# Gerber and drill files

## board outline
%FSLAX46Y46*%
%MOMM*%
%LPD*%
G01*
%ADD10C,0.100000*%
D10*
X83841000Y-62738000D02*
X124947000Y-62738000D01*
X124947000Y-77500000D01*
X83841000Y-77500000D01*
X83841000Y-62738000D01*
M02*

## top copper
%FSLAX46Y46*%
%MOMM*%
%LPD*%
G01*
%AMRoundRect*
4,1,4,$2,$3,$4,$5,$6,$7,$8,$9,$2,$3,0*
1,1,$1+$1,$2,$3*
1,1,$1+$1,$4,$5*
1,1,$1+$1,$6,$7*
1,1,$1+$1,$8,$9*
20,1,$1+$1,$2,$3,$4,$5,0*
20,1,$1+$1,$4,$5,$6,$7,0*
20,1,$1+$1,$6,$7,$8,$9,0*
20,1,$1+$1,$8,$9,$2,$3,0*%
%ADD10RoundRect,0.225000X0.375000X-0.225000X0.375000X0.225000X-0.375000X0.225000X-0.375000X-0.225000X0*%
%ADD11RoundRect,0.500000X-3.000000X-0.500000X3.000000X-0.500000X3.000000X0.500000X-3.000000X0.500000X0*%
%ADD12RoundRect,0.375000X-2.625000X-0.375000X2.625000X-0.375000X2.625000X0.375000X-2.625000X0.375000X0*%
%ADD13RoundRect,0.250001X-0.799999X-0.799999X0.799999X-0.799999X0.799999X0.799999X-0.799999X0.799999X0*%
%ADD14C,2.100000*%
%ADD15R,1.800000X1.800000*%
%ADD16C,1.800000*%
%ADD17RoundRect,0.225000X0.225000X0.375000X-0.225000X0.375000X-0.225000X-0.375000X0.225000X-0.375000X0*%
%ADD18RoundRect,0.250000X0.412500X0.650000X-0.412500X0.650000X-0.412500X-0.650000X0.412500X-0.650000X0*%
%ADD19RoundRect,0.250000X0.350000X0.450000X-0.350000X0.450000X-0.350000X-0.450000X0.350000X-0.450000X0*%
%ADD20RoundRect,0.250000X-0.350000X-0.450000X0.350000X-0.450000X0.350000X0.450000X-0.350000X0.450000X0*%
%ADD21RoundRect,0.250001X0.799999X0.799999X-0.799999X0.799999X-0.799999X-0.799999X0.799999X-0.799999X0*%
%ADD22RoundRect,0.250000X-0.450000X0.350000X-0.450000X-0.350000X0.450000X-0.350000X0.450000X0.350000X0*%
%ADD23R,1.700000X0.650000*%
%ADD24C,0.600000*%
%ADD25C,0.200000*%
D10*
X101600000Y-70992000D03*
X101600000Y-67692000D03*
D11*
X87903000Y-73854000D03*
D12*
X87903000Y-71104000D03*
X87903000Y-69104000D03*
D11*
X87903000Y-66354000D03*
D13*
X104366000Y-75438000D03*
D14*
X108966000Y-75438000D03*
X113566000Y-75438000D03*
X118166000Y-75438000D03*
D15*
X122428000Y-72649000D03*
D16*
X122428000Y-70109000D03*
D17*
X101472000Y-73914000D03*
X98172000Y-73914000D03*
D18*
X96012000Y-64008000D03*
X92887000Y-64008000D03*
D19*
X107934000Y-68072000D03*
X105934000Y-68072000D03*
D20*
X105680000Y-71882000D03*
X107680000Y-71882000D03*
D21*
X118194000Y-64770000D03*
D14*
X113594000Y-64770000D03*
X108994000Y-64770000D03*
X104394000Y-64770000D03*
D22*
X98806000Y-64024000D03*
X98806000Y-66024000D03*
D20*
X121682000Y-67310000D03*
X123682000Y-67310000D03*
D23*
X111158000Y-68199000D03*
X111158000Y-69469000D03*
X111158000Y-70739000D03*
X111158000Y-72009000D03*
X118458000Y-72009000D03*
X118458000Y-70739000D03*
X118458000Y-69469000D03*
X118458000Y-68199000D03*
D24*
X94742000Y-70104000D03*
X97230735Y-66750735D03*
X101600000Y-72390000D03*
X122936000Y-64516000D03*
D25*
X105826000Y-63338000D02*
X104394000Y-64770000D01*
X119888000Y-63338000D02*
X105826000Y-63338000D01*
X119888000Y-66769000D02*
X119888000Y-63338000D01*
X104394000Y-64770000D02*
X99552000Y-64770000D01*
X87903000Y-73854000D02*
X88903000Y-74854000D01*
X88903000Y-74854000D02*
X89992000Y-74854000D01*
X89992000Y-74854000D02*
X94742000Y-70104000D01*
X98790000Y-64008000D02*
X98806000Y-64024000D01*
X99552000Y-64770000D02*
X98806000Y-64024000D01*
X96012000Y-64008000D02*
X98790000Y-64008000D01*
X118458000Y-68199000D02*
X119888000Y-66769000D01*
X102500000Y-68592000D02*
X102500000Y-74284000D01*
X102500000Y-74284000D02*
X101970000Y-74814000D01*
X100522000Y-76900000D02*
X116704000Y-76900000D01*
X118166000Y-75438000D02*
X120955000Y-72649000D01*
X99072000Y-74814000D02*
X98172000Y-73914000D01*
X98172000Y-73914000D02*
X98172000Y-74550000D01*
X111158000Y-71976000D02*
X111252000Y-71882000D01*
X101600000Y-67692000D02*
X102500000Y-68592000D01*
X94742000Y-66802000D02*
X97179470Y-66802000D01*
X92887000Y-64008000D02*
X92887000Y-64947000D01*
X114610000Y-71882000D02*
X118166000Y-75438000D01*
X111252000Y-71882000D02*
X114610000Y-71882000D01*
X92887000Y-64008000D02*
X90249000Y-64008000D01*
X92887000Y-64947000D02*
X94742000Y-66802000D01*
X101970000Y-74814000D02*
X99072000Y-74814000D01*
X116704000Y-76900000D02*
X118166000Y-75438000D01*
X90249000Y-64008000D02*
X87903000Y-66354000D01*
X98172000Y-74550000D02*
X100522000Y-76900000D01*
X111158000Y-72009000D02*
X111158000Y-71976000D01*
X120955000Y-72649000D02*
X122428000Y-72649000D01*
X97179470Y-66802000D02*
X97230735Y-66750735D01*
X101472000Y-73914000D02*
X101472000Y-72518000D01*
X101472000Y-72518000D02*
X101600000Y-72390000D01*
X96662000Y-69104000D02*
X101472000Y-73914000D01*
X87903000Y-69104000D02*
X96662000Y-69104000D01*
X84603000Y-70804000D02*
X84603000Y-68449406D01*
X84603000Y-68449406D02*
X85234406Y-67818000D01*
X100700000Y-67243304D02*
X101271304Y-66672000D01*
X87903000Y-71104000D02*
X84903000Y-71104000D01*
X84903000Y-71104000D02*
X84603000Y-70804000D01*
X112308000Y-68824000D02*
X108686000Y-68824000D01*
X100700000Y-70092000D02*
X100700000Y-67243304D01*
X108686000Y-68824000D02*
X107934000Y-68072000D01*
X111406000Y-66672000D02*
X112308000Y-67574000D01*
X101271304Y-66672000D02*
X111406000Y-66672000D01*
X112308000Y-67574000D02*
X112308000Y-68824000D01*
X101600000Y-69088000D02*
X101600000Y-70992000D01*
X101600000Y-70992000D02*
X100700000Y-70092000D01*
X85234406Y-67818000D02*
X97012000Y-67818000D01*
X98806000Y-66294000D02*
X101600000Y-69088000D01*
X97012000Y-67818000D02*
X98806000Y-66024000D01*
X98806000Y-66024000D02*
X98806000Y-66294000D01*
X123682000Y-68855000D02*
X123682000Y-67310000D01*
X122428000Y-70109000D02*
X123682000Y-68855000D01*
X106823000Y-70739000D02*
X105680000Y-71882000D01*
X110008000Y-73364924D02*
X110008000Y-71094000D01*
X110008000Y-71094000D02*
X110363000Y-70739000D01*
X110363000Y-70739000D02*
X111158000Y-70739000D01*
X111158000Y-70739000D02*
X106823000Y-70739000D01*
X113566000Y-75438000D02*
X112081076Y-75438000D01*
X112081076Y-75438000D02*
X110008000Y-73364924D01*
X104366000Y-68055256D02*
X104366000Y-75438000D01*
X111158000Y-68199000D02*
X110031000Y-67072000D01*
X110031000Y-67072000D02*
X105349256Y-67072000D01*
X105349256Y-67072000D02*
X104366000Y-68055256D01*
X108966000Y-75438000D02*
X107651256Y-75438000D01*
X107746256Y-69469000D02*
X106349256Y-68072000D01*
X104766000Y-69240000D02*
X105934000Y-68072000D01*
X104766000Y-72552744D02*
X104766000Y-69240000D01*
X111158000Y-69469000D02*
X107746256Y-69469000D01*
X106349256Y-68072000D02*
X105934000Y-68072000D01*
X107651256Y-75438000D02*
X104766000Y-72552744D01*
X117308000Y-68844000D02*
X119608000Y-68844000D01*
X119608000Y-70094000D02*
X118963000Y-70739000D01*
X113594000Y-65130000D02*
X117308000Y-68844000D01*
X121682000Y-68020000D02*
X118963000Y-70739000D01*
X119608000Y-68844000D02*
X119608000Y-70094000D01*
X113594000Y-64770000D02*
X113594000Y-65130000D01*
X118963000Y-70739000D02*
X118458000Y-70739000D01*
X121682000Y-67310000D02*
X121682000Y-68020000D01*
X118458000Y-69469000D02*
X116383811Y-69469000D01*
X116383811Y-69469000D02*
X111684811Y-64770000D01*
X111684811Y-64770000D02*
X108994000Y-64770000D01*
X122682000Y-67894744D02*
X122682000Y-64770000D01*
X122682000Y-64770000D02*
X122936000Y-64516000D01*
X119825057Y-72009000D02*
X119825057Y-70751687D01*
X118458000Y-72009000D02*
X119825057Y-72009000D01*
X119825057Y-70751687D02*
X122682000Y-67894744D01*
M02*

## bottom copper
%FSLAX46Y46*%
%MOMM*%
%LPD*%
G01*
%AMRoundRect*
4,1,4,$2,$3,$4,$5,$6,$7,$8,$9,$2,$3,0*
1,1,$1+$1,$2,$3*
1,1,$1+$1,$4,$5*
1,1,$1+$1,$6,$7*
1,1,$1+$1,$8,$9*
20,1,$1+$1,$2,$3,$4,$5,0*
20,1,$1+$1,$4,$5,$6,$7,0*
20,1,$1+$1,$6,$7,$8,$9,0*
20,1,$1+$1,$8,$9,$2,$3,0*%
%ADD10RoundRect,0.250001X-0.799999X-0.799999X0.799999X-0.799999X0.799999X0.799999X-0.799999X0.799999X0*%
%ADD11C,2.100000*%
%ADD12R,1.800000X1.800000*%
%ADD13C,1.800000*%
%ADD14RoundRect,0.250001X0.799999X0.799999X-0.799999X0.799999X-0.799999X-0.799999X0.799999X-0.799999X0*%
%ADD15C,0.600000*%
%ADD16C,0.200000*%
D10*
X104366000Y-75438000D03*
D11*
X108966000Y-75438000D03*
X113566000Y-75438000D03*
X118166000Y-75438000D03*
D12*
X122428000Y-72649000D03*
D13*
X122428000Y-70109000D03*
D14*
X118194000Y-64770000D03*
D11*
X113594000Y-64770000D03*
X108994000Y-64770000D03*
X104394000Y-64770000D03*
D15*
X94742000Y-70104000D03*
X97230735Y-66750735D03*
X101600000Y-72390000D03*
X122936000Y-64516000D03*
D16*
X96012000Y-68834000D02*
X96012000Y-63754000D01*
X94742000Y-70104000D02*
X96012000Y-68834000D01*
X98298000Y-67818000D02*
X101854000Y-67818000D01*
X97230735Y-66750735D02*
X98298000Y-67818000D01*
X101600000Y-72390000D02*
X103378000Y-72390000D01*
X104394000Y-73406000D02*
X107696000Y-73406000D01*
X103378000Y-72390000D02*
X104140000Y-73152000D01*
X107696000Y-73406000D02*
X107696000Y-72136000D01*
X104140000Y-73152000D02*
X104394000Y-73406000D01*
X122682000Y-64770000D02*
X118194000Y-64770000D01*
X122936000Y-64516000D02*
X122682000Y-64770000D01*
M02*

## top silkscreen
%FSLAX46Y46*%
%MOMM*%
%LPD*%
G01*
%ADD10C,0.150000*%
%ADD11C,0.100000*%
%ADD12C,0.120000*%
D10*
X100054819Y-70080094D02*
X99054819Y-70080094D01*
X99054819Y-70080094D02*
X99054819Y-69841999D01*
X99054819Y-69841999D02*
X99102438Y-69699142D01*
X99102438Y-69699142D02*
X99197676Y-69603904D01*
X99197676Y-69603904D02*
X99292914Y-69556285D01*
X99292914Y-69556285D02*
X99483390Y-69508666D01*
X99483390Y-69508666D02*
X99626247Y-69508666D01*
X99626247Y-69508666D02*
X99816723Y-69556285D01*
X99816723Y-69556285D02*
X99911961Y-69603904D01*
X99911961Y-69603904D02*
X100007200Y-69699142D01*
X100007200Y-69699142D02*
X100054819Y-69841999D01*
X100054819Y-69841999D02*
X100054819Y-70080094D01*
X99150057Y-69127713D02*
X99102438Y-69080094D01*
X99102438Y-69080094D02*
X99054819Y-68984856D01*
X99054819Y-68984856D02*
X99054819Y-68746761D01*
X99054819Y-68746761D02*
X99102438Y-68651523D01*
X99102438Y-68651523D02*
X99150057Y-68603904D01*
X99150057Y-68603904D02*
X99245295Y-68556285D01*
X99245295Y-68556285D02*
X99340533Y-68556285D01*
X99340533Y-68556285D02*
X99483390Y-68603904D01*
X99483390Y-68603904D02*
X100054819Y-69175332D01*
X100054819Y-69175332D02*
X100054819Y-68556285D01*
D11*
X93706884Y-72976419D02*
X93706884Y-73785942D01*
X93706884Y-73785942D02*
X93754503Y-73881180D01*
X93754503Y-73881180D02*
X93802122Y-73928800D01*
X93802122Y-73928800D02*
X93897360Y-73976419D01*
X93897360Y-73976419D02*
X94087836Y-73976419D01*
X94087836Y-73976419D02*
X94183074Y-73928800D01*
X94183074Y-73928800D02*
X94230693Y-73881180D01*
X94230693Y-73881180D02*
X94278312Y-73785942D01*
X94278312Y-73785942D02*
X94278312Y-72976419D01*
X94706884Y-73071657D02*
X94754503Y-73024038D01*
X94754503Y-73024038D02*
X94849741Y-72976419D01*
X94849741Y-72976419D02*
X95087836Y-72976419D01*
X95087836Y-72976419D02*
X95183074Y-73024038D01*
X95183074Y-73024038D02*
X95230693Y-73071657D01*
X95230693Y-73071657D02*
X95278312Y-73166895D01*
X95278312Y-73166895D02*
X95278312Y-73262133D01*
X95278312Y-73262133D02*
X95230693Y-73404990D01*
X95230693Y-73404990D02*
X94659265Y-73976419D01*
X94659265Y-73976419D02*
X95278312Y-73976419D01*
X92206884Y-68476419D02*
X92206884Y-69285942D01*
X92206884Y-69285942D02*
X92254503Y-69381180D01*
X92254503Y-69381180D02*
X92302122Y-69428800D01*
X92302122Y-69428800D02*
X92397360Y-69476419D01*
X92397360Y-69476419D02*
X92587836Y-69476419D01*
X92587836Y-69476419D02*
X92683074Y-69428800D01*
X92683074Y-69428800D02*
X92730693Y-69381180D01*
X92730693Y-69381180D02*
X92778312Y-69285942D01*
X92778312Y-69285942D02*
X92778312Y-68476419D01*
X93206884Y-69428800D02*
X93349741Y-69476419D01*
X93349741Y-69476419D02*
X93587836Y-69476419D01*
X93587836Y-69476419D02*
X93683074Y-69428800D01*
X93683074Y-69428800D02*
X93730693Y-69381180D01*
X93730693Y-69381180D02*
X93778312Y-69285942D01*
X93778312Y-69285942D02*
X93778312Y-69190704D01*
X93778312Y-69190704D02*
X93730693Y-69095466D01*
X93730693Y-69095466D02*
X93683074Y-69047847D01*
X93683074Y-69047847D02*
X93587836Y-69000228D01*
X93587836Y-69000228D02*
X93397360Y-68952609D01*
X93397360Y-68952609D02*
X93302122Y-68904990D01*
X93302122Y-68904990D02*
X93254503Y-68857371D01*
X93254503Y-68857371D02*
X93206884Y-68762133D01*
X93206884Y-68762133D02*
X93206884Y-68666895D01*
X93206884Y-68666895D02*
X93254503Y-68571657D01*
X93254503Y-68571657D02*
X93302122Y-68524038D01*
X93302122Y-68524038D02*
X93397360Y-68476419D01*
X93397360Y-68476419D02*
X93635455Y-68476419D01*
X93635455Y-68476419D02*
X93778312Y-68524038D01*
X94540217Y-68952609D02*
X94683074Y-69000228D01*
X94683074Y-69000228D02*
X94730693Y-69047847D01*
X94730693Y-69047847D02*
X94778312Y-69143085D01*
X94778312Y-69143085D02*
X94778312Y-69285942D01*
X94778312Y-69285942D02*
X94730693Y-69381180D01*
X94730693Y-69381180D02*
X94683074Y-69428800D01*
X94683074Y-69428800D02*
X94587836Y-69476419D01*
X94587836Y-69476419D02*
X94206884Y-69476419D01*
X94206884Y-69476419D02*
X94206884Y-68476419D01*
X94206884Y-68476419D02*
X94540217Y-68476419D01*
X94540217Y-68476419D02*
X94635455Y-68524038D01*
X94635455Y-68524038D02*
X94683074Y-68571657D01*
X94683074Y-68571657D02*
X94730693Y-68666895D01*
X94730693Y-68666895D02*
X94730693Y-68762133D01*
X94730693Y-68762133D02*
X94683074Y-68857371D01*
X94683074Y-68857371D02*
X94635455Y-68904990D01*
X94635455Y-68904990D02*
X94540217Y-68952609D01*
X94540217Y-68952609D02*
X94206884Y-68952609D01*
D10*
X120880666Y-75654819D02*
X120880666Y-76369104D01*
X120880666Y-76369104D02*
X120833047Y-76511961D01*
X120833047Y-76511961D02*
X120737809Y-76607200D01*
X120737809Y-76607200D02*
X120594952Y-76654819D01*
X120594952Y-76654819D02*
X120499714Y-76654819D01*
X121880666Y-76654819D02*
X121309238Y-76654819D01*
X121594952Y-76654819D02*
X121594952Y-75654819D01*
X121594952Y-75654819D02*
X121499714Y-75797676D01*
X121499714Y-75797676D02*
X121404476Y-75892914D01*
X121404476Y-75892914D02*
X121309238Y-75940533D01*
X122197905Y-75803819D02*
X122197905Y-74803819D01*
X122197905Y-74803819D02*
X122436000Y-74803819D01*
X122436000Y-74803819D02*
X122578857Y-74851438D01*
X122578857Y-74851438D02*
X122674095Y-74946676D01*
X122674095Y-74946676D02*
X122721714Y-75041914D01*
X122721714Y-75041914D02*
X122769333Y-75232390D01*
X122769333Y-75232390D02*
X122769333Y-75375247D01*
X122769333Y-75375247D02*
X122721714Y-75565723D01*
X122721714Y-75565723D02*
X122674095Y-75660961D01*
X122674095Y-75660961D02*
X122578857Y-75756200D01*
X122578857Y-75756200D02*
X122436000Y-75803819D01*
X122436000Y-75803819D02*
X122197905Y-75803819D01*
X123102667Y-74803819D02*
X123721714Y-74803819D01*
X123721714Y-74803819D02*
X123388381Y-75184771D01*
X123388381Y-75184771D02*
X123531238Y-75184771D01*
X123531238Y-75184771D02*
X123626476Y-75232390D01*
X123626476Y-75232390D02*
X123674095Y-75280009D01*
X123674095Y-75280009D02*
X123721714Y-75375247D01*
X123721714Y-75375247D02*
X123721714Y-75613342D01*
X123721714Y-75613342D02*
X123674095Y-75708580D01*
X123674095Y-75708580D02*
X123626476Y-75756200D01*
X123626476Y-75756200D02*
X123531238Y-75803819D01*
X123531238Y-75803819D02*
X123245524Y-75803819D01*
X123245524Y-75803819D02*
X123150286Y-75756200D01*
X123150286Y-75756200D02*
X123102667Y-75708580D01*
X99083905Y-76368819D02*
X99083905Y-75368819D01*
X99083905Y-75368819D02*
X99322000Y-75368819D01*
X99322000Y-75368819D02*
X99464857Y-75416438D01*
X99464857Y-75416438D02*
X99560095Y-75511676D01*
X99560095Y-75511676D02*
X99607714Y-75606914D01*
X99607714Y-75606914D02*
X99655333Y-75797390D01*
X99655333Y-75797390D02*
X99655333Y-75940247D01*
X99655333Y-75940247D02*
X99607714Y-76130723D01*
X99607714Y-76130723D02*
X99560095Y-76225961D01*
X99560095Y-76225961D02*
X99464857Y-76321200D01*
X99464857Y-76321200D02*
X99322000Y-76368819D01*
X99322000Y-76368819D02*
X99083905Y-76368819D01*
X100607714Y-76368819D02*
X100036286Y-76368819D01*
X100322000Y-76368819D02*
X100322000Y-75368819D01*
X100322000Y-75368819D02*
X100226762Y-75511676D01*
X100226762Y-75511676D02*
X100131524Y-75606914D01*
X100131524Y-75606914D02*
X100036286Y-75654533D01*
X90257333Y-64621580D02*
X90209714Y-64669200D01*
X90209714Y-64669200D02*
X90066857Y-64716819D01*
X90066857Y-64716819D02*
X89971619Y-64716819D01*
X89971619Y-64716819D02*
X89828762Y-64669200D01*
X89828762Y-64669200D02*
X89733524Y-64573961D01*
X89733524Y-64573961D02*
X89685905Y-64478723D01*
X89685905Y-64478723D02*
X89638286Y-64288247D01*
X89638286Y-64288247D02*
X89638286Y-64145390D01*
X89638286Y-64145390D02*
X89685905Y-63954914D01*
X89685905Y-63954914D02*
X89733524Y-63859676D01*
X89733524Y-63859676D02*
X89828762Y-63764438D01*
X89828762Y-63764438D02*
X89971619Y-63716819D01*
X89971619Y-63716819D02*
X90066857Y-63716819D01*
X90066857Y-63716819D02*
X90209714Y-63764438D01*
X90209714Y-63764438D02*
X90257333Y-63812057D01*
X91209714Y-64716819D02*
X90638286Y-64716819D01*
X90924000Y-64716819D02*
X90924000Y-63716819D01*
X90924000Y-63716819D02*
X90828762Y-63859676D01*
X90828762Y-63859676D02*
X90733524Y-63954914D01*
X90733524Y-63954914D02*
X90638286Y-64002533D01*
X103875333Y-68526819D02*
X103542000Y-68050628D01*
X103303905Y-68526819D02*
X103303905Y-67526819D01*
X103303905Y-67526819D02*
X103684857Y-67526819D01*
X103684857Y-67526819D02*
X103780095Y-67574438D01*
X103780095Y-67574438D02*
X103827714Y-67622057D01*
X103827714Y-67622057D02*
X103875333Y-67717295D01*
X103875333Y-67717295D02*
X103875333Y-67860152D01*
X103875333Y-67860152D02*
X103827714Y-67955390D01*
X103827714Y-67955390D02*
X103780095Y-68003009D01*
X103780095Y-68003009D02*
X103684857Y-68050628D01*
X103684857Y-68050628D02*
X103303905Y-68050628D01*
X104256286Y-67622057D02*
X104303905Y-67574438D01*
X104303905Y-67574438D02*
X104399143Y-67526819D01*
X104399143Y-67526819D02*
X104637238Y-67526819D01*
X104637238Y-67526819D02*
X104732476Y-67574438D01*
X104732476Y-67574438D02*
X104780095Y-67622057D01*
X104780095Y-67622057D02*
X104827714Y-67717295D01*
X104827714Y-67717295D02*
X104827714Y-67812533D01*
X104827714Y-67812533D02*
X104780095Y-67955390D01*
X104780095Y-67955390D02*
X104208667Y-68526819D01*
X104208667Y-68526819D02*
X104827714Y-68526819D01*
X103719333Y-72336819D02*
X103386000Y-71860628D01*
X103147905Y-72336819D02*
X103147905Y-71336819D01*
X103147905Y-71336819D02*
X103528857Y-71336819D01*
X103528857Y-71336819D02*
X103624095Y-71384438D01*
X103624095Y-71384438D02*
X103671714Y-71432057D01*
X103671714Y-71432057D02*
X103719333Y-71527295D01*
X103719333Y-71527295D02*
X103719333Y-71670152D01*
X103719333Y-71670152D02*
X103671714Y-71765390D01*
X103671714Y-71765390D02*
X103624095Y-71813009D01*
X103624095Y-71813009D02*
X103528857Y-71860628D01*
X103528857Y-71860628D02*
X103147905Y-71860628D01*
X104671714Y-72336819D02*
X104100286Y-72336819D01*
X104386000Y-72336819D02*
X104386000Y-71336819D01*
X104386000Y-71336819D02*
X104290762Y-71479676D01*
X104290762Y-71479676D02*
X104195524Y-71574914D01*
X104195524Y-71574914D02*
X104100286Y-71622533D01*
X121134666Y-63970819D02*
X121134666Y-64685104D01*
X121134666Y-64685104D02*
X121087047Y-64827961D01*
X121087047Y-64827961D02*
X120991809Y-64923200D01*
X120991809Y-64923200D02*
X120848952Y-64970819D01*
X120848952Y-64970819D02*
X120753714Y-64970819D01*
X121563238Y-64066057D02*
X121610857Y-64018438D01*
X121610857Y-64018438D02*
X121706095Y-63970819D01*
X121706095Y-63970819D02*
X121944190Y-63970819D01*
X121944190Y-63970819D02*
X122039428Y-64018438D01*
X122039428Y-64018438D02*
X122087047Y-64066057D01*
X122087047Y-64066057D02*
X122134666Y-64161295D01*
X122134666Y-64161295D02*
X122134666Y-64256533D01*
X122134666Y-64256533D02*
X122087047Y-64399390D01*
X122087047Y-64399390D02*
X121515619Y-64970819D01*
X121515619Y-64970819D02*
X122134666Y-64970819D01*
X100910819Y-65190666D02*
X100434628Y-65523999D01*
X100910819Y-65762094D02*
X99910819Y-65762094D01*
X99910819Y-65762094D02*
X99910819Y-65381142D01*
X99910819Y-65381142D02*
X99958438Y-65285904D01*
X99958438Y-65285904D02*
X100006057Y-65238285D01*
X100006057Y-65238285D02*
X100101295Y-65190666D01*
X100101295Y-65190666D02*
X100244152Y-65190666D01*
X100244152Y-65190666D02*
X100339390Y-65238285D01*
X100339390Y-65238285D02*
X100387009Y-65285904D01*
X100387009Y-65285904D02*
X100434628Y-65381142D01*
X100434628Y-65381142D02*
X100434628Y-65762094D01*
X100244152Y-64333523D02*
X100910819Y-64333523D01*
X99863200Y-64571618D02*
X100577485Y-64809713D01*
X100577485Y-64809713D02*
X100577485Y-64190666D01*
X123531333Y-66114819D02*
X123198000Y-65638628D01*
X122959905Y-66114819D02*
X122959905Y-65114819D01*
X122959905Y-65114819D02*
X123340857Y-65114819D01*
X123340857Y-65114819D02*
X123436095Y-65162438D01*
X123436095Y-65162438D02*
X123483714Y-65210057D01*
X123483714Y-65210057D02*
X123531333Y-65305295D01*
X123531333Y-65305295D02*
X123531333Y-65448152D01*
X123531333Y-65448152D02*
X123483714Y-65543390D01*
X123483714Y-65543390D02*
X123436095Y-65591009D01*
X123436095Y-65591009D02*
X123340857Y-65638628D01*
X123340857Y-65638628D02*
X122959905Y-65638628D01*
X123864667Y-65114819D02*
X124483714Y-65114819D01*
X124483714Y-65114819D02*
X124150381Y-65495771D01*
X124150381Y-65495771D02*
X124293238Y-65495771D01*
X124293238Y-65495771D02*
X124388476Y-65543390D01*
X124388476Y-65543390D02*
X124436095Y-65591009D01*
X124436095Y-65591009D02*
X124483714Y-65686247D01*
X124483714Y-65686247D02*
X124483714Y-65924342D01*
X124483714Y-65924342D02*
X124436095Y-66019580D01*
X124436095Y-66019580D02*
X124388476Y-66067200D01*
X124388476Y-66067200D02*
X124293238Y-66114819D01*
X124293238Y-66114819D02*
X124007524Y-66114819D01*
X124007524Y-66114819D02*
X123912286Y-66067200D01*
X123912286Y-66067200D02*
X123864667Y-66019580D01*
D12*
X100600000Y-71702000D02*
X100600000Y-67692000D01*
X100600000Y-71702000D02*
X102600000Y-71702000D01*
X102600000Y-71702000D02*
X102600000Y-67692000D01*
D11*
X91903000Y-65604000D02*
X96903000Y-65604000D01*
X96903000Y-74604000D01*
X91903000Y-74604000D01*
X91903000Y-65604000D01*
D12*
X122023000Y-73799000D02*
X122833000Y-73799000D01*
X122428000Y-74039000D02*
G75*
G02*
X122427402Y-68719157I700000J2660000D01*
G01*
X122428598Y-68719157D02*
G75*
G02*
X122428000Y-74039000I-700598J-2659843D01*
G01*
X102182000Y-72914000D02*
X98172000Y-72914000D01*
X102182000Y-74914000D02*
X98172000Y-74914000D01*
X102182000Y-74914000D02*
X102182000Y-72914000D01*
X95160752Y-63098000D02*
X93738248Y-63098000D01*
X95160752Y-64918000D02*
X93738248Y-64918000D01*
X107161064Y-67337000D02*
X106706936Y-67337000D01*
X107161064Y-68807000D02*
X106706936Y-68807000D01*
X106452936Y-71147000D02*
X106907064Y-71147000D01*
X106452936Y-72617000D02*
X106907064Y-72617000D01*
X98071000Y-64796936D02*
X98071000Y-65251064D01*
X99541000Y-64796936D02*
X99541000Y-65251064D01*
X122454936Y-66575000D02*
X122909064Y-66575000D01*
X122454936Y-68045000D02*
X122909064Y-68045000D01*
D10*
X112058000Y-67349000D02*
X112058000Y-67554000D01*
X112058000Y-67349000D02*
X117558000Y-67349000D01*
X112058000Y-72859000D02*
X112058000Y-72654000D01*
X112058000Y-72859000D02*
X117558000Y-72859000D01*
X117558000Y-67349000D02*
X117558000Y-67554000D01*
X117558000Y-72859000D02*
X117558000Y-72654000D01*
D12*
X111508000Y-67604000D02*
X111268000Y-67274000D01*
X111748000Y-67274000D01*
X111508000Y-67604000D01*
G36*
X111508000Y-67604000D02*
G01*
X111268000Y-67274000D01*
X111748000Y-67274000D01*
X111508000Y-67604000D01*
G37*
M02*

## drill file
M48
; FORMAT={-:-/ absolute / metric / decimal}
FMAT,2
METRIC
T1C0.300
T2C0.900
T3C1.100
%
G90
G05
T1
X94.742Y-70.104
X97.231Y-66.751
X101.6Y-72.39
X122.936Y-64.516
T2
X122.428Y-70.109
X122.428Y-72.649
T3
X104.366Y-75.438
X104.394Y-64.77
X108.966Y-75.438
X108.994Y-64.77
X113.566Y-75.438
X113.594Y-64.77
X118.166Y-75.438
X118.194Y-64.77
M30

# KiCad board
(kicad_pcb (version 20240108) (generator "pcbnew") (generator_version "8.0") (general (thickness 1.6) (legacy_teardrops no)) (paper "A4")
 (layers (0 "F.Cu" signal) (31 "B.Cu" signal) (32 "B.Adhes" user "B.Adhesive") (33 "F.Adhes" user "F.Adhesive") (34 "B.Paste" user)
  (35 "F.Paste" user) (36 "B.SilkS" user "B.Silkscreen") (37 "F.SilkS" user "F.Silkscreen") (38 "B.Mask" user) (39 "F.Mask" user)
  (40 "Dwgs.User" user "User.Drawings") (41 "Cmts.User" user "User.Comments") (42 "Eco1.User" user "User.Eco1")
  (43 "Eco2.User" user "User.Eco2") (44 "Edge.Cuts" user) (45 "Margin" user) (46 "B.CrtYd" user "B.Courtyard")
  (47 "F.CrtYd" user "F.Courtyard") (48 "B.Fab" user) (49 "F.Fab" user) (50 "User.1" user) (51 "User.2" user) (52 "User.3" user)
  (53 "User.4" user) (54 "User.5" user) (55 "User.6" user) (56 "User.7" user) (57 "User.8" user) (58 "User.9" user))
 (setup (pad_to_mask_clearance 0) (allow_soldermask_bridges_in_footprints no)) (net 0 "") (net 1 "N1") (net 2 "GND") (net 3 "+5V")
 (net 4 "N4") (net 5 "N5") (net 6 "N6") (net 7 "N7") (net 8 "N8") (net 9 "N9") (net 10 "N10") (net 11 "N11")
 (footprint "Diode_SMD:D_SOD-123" (layer "F.Cu") (at 101.6 69.342 90)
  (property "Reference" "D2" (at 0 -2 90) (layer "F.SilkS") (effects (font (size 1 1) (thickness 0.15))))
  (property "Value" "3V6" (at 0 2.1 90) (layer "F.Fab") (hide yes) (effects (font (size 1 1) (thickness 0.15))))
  (fp_line (start -2.36 -1) (end 1.65 -1) (stroke (width 0.12) (type solid)) (layer "F.SilkS"))
  (fp_line (start -2.36 -1) (end -2.36 1) (stroke (width 0.12) (type solid)) (layer "F.SilkS"))
  (fp_line (start -2.36 1) (end 1.65 1) (stroke (width 0.12) (type solid)) (layer "F.SilkS"))
  (pad "1" smd roundrect (at -1.65 0 90) (size 0.9 1.2) (layers "F.Cu" "F.Paste" "F.Mask") (roundrect_rratio 0.25) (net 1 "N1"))
  (pad "2" smd roundrect (at 1.65 0 90) (size 0.9 1.2) (layers "F.Cu" "F.Paste" "F.Mask") (roundrect_rratio 0.25) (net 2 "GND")))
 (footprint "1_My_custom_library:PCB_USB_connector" (layer "F.Cu") (at 87.903 70.104)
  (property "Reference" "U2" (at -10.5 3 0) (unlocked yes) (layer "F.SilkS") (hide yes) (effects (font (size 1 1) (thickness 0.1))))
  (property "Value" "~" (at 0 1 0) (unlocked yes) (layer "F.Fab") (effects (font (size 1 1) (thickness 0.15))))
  (fp_rect (start 4 -4.5) (end 9 4.5) (stroke (width 0.1) (type default)) (fill none) (layer "F.SilkS"))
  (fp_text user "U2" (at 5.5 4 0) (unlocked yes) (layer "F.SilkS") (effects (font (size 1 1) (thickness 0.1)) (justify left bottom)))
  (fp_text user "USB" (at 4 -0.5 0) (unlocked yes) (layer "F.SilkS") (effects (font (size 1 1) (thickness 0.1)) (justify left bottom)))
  (pad "1" smd roundrect (at 0 3.75) (size 7 2) (layers "F.Cu" "F.Paste" "F.Mask") (roundrect_rratio 0.25) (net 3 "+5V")
   (thermal_bridge_angle 45))
  (pad "2" smd roundrect (at 0 1) (size 6 1.5) (layers "F.Cu" "F.Paste" "F.Mask") (roundrect_rratio 0.25) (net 1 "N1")
   (thermal_bridge_angle 45))
  (pad "3" smd roundrect (at 0 -1) (size 6 1.5) (layers "F.Cu" "F.Paste" "F.Mask") (roundrect_rratio 0.25) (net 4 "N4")
   (thermal_bridge_angle 45))
  (pad "4" smd roundrect (at 0 -3.75) (size 7 2) (layers "F.Cu" "F.Paste" "F.Mask") (roundrect_rratio 0.25) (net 2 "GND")
   (thermal_bridge_angle 45)))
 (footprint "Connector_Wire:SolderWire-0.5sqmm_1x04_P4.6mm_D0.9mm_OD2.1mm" (layer "F.Cu") (at 104.366 75.438)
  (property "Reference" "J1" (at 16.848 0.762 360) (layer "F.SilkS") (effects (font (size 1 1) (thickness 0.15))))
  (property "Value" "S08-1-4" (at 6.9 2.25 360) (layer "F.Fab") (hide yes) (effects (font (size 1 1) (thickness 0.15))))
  (pad "1" thru_hole roundrect (at 0 0) (size 2.1 2.1) (drill 1.1) (layers "*.Cu" "*.Mask") (remove_unused_layers no)
   (roundrect_rratio 0.119048) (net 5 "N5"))
  (pad "2" thru_hole circle (at 4.6 0) (size 2.1 2.1) (drill 1.1) (layers "*.Cu" "*.Mask") (remove_unused_layers no) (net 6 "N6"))
  (pad "3" thru_hole circle (at 9.2 0) (size 2.1 2.1) (drill 1.1) (layers "*.Cu" "*.Mask") (remove_unused_layers no) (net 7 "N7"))
  (pad "4" thru_hole circle (at 13.8 0) (size 2.1 2.1) (drill 1.1) (layers "*.Cu" "*.Mask") (remove_unused_layers no) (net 2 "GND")))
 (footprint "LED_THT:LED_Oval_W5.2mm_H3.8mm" (layer "F.Cu") (at 122.428 72.649 90)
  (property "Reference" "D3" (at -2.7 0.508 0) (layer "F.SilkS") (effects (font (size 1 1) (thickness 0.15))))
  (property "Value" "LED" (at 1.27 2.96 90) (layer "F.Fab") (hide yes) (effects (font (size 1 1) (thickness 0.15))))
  (fp_line (start -1.15 -0.405) (end -1.15 0.405) (stroke (width 0.12) (type solid)) (layer "F.SilkS"))
  (fp_arc (start -1.39 0) (mid 1.269691 -2.050564) (end 3.929843 -0.000598) (stroke (width 0.12) (type solid)) (layer "F.SilkS"))
  (fp_arc (start 3.929843 0.000598) (mid 1.269691 2.050564) (end -1.39 0) (stroke (width 0.12) (type solid)) (layer "F.SilkS"))
  (pad "1" thru_hole rect (at 0 0 90) (size 1.8 1.8) (drill 0.9) (layers "*.Cu" "*.Mask") (remove_unused_layers no) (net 2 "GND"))
  (pad "2" thru_hole circle (at 2.54 0 90) (size 1.8 1.8) (drill 0.9) (layers "*.Cu" "*.Mask") (remove_unused_layers no) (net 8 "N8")))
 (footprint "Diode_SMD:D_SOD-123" (layer "F.Cu") (at 99.822 73.914 180)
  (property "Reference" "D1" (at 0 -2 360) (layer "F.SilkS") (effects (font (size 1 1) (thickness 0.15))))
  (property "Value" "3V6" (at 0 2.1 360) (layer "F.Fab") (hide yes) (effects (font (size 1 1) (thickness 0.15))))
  (fp_line (start -2.36 1) (end 1.65 1) (stroke (width 0.12) (type solid)) (layer "F.SilkS"))
  (fp_line (start -2.36 -1) (end 1.65 -1) (stroke (width 0.12) (type solid)) (layer "F.SilkS"))
  (fp_line (start -2.36 -1) (end -2.36 1) (stroke (width 0.12) (type solid)) (layer "F.SilkS"))
  (pad "1" smd roundrect (at -1.65 0 180) (size 0.9 1.2) (layers "F.Cu" "F.Paste" "F.Mask") (roundrect_rratio 0.25) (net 4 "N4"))
  (pad "2" smd roundrect (at 1.65 0 180) (size 0.9 1.2) (layers "F.Cu" "F.Paste" "F.Mask") (roundrect_rratio 0.25) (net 2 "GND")))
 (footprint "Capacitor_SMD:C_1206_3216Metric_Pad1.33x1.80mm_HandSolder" (layer "F.Cu") (at 94.4495 64.008 180)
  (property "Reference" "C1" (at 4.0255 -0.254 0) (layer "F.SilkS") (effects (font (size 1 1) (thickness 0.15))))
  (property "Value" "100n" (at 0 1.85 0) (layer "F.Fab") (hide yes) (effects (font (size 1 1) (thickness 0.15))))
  (fp_line (start -0.711252 0.91) (end 0.711252 0.91) (stroke (width 0.12) (type solid)) (layer "F.SilkS"))
  (fp_line (start -0.711252 -0.91) (end 0.711252 -0.91) (stroke (width 0.12) (type solid)) (layer "F.SilkS"))
  (pad "1" smd roundrect (at -1.5625 0 180) (size 1.325 1.8) (layers "F.Cu" "F.Paste" "F.Mask") (roundrect_rratio 0.188679) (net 3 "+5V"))
  (pad "2" smd roundrect (at 1.5625 0 180) (size 1.325 1.8) (layers "F.Cu" "F.Paste" "F.Mask") (roundrect_rratio 0.188679) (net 2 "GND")))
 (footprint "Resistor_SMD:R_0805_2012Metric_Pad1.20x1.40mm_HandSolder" (layer "F.Cu") (at 106.934 68.072 180)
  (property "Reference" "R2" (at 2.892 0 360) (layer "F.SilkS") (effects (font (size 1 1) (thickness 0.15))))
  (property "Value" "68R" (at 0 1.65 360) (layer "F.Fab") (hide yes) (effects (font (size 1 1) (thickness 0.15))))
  (fp_line (start -0.227064 0.735) (end 0.227064 0.735) (stroke (width 0.12) (type solid)) (layer "F.SilkS"))
  (fp_line (start -0.227064 -0.735) (end 0.227064 -0.735) (stroke (width 0.12) (type solid)) (layer "F.SilkS"))
  (pad "1" smd roundrect (at -1 0 180) (size 1.2 1.4) (layers "F.Cu" "F.Paste" "F.Mask") (roundrect_rratio 0.208333) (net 1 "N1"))
  (pad "2" smd roundrect (at 1 0 180) (size 1.2 1.4) (layers "F.Cu" "F.Paste" "F.Mask") (roundrect_rratio 0.208333) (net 6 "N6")))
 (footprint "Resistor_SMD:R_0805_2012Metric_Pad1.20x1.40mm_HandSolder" (layer "F.Cu") (at 106.68 71.882)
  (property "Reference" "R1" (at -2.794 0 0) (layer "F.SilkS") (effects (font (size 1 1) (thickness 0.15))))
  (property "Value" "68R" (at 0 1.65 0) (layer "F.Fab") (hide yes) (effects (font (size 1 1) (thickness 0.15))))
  (fp_line (start -0.227064 -0.735) (end 0.227064 -0.735) (stroke (width 0.12) (type solid)) (layer "F.SilkS"))
  (fp_line (start -0.227064 0.735) (end 0.227064 0.735) (stroke (width 0.12) (type solid)) (layer "F.SilkS"))
  (pad "1" smd roundrect (at -1 0) (size 1.2 1.4) (layers "F.Cu" "F.Paste" "F.Mask") (roundrect_rratio 0.208333) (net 7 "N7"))
  (pad "2" smd roundrect (at 1 0) (size 1.2 1.4) (layers "F.Cu" "F.Paste" "F.Mask") (roundrect_rratio 0.208333) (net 4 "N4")))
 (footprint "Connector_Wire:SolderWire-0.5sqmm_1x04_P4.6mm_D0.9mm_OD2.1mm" (layer "F.Cu") (at 118.194 64.77 180)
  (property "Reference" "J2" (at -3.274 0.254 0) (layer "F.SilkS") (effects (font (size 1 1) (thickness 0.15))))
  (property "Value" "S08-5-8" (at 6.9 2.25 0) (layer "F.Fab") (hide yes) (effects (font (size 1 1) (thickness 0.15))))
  (pad "1" thru_hole roundrect (at 0 0 180) (size 2.1 2.1) (drill 1.1) (layers "*.Cu" "*.Mask") (remove_unused_layers no)
   (roundrect_rratio 0.119048) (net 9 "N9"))
  (pad "2" thru_hole circle (at 4.6 0 180) (size 2.1 2.1) (drill 1.1) (layers "*.Cu" "*.Mask") (remove_unused_layers no) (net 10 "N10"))
  (pad "3" thru_hole circle (at 9.2 0 180) (size 2.1 2.1) (drill 1.1) (layers "*.Cu" "*.Mask") (remove_unused_layers no) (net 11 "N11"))
  (pad "4" thru_hole circle (at 13.8 0 180) (size 2.1 2.1) (drill 1.1) (layers "*.Cu" "*.Mask") (remove_unused_layers no) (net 3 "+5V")))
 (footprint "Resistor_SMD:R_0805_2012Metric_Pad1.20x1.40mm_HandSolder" (layer "F.Cu") (at 98.806 65.024 -90)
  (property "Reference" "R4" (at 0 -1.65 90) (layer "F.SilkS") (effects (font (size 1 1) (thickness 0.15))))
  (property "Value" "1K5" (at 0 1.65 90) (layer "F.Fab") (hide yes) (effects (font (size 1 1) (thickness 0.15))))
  (fp_line (start -0.227064 0.735) (end 0.227064 0.735) (stroke (width 0.12) (type solid)) (layer "F.SilkS"))
  (fp_line (start -0.227064 -0.735) (end 0.227064 -0.735) (stroke (width 0.12) (type solid)) (layer "F.SilkS"))
  (pad "1" smd roundrect (at -1 0 270) (size 1.2 1.4) (layers "F.Cu" "F.Paste" "F.Mask") (roundrect_rratio 0.208333) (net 3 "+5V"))
  (pad "2" smd roundrect (at 1 0 270) (size 1.2 1.4) (layers "F.Cu" "F.Paste" "F.Mask") (roundrect_rratio 0.208333) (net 1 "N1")))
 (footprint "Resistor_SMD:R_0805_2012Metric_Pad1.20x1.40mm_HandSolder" (layer "F.Cu") (at 122.682 67.31)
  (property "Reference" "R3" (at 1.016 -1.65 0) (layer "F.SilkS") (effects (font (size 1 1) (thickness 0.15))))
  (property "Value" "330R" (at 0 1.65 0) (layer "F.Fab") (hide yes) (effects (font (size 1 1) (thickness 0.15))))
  (fp_line (start -0.227064 -0.735) (end 0.227064 -0.735) (stroke (width 0.12) (type solid)) (layer "F.SilkS"))
  (fp_line (start -0.227064 0.735) (end 0.227064 0.735) (stroke (width 0.12) (type solid)) (layer "F.SilkS"))
  (pad "1" smd roundrect (at -1 0) (size 1.2 1.4) (layers "F.Cu" "F.Paste" "F.Mask") (roundrect_rratio 0.208333) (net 10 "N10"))
  (pad "2" smd roundrect (at 1 0) (size 1.2 1.4) (layers "F.Cu" "F.Paste" "F.Mask") (roundrect_rratio 0.208333) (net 8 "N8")))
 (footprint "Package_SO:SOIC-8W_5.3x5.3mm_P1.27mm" (layer "F.Cu") (at 114.808 70.104)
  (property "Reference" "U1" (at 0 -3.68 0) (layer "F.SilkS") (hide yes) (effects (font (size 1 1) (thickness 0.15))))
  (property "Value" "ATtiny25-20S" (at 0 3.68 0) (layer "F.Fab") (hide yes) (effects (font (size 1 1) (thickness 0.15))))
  (fp_line (start -2.75 -2.755) (end -2.75 -2.55) (stroke (width 0.15) (type solid)) (layer "F.SilkS"))
  (fp_line (start -2.75 -2.755) (end 2.75 -2.755) (stroke (width 0.15) (type solid)) (layer "F.SilkS"))
  (fp_line (start -2.75 2.755) (end -2.75 2.55) (stroke (width 0.15) (type solid)) (layer "F.SilkS"))
  (fp_line (start -2.75 2.755) (end 2.75 2.755) (stroke (width 0.15) (type solid)) (layer "F.SilkS"))
  (fp_line (start 2.75 -2.755) (end 2.75 -2.55) (stroke (width 0.15) (type solid)) (layer "F.SilkS"))
  (fp_line (start 2.75 2.755) (end 2.75 2.55) (stroke (width 0.15) (type solid)) (layer "F.SilkS"))
  (fp_poly
   (pts (xy -3.3 -2.5) (xy -3.54 -2.83) (xy -3.06 -2.83) (xy -3.3 -2.5)) (stroke (width 0.12) (type solid)) (fill solid) (layer "F.SilkS"))
  (pad "1" smd rect (at -3.65 -1.905) (size 1.7 0.65) (layers "F.Cu" "F.Paste" "F.Mask") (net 5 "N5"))
  (pad "2" smd rect (at -3.65 -0.635) (size 1.7 0.65) (layers "F.Cu" "F.Paste" "F.Mask") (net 6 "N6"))
  (pad "3" smd rect (at -3.65 0.635) (size 1.7 0.65) (layers "F.Cu" "F.Paste" "F.Mask") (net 7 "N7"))
  (pad "4" smd rect (at -3.65 1.905) (size 1.7 0.65) (layers "F.Cu" "F.Paste" "F.Mask") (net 2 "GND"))
  (pad "5" smd rect (at 3.65 1.905) (size 1.7 0.65) (layers "F.Cu" "F.Paste" "F.Mask") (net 9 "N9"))
  (pad "6" smd rect (at 3.65 0.635) (size 1.7 0.65) (layers "F.Cu" "F.Paste" "F.Mask") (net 10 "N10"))
  (pad "7" smd rect (at 3.65 -0.635) (size 1.7 0.65) (layers "F.Cu" "F.Paste" "F.Mask") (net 11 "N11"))
  (pad "8" smd rect (at 3.65 -1.905) (size 1.7 0.65) (layers "F.Cu" "F.Paste" "F.Mask") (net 3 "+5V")))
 (gr_rect (start 83.841 62.738) (end 124.947 77.5) (stroke (width 0.1) (type default)) (fill none) (layer "Edge.Cuts"))
 (segment (start 105.826 63.338) (end 104.394 64.77) (width 0.2) (layer "F.Cu") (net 3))
 (segment (start 119.888 63.338) (end 105.826 63.338) (width 0.2) (layer "F.Cu") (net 3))
 (segment (start 119.888 66.769) (end 119.888 63.338) (width 0.2) (layer "F.Cu") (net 3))
 (segment (start 104.394 64.77) (end 99.552 64.77) (width 0.2) (layer "F.Cu") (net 3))
 (segment (start 87.903 73.854) (end 88.903 74.854) (width 0.2) (layer "F.Cu") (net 3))
 (segment (start 88.903 74.854) (end 89.992 74.854) (width 0.2) (layer "F.Cu") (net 3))
 (segment (start 89.992 74.854) (end 94.742 70.104) (width 0.2) (layer "F.Cu") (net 3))
 (segment (start 98.79 64.008) (end 98.806 64.024) (width 0.2) (layer "F.Cu") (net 3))
 (segment (start 99.552 64.77) (end 98.806 64.024) (width 0.2) (layer "F.Cu") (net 3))
 (segment (start 96.012 64.008) (end 98.79 64.008) (width 0.2) (layer "F.Cu") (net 3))
 (segment (start 118.458 68.199) (end 119.888 66.769) (width 0.2) (layer "F.Cu") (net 3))
 (via (at 94.742 70.104) (size 0.6) (drill 0.3) (layers "F.Cu" "B.Cu") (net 3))
 (segment (start 96.012 68.834) (end 96.012 63.754) (width 0.2) (layer "B.Cu") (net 3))
 (segment (start 94.742 70.104) (end 96.012 68.834) (width 0.2) (layer "B.Cu") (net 3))
 (segment (start 102.5 68.592) (end 102.5 74.284) (width 0.2) (layer "F.Cu") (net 2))
 (segment (start 102.5 74.284) (end 101.97 74.814) (width 0.2) (layer "F.Cu") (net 2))
 (segment (start 100.522 76.9) (end 116.704 76.9) (width 0.2) (layer "F.Cu") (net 2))
 (segment (start 118.166 75.438) (end 120.955 72.649) (width 0.2) (layer "F.Cu") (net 2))
 (segment (start 99.072 74.814) (end 98.172 73.914) (width 0.2) (layer "F.Cu") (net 2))
 (segment (start 98.172 73.914) (end 98.172 74.55) (width 0.2) (layer "F.Cu") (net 2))
 (segment (start 111.158 71.976) (end 111.252 71.882) (width 0.2) (layer "F.Cu") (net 2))
 (segment (start 101.6 67.692) (end 102.5 68.592) (width 0.2) (layer "F.Cu") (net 2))
 (segment (start 94.742 66.802) (end 97.17947 66.802) (width 0.2) (layer "F.Cu") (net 2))
 (segment (start 92.887 64.008) (end 92.887 64.947) (width 0.2) (layer "F.Cu") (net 2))
 (segment (start 114.61 71.882) (end 118.166 75.438) (width 0.2) (layer "F.Cu") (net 2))
 (segment (start 111.252 71.882) (end 114.61 71.882) (width 0.2) (layer "F.Cu") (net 2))
 (segment (start 92.887 64.008) (end 90.249 64.008) (width 0.2) (layer "F.Cu") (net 2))
 (segment (start 92.887 64.947) (end 94.742 66.802) (width 0.2) (layer "F.Cu") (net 2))
 (segment (start 101.97 74.814) (end 99.072 74.814) (width 0.2) (layer "F.Cu") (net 2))
 (segment (start 116.704 76.9) (end 118.166 75.438) (width 0.2) (layer "F.Cu") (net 2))
 (segment (start 90.249 64.008) (end 87.903 66.354) (width 0.2) (layer "F.Cu") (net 2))
 (segment (start 98.172 74.55) (end 100.522 76.9) (width 0.2) (layer "F.Cu") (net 2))
 (segment (start 111.158 72.009) (end 111.158 71.976) (width 0.2) (layer "F.Cu") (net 2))
 (segment (start 120.955 72.649) (end 122.428 72.649) (width 0.2) (layer "F.Cu") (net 2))
 (segment (start 97.17947 66.802) (end 97.230735 66.750735) (width 0.2) (layer "F.Cu") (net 2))
 (via (at 97.230735 66.750735) (size 0.6) (drill 0.3) (layers "F.Cu" "B.Cu") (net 2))
 (segment (start 98.298 67.818) (end 101.854 67.818) (width 0.2) (layer "B.Cu") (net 2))
 (segment (start 97.230735 66.750735) (end 98.298 67.818) (width 0.2) (layer "B.Cu") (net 2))
 (segment (start 101.472 73.914) (end 101.472 72.518) (width 0.2) (layer "F.Cu") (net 4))
 (segment (start 101.472 72.518) (end 101.6 72.39) (width 0.2) (layer "F.Cu") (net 4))
 (segment (start 96.662 69.104) (end 101.472 73.914) (width 0.2) (layer "F.Cu") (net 4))
 (segment (start 87.903 69.104) (end 96.662 69.104) (width 0.2) (layer "F.Cu") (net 4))
 (via (at 101.6 72.39) (size 0.6) (drill 0.3) (layers "F.Cu" "B.Cu") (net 4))
 (segment (start 101.6 72.39) (end 103.378 72.39) (width 0.2) (layer "B.Cu") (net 4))
 (segment (start 104.394 73.406) (end 107.696 73.406) (width 0.2) (layer "B.Cu") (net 4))
 (segment (start 103.378 72.39) (end 104.14 73.152) (width 0.2) (layer "B.Cu") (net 4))
 (segment (start 107.696 73.406) (end 107.696 72.136) (width 0.2) (layer "B.Cu") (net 4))
 (segment (start 104.14 73.152) (end 104.394 73.406) (width 0.2) (layer "B.Cu") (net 4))
 (segment (start 84.603 70.804) (end 84.603 68.449406) (width 0.2) (layer "F.Cu") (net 1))
 (segment (start 84.603 68.449406) (end 85.234406 67.818) (width 0.2) (layer "F.Cu") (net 1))
 (segment (start 100.7 67.243304) (end 101.271304 66.672) (width 0.2) (layer "F.Cu") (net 1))
 (segment (start 87.903 71.104) (end 84.903 71.104) (width 0.2) (layer "F.Cu") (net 1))
 (segment (start 84.903 71.104) (end 84.603 70.804) (width 0.2) (layer "F.Cu") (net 1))
 (segment (start 112.308 68.824) (end 108.686 68.824) (width 0.2) (layer "F.Cu") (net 1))
 (segment (start 100.7 70.092) (end 100.7 67.243304) (width 0.2) (layer "F.Cu") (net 1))
 (segment (start 108.686 68.824) (end 107.934 68.072) (width 0.2) (layer "F.Cu") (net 1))
 (segment (start 111.406 66.672) (end 112.308 67.574) (width 0.2) (layer "F.Cu") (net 1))
 (segment (start 101.271304 66.672) (end 111.406 66.672) (width 0.2) (layer "F.Cu") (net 1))
 (segment (start 112.308 67.574) (end 112.308 68.824) (width 0.2) (layer "F.Cu") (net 1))
 (segment (start 101.6 69.088) (end 101.6 70.992) (width 0.2) (layer "F.Cu") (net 1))
 (segment (start 101.6 70.992) (end 100.7 70.092) (width 0.2) (layer "F.Cu") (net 1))
 (segment (start 85.234406 67.818) (end 97.012 67.818) (width 0.2) (layer "F.Cu") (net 1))
 (segment (start 98.806 66.294) (end 101.6 69.088) (width 0.2) (layer "F.Cu") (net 1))
 (segment (start 97.012 67.818) (end 98.806 66.024) (width 0.2) (layer "F.Cu") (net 1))
 (segment (start 98.806 66.024) (end 98.806 66.294) (width 0.2) (layer "F.Cu") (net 1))
 (segment (start 123.682 68.855) (end 123.682 67.31) (width 0.2) (layer "F.Cu") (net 8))
 (segment (start 122.428 70.109) (end 123.682 68.855) (width 0.2) (layer "F.Cu") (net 8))
 (segment (start 106.823 70.739) (end 105.68 71.882) (width 0.2) (layer "F.Cu") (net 7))
 (segment (start 110.008 73.364924) (end 110.008 71.094) (width 0.2) (layer "F.Cu") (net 7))
 (segment (start 110.008 71.094) (end 110.363 70.739) (width 0.2) (layer "F.Cu") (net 7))
 (segment (start 110.363 70.739) (end 111.158 70.739) (width 0.2) (layer "F.Cu") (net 7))
 (segment (start 111.158 70.739) (end 106.823 70.739) (width 0.2) (layer "F.Cu") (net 7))
 (segment (start 113.566 75.438) (end 112.081076 75.438) (width 0.2) (layer "F.Cu") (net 7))
 (segment (start 112.081076 75.438) (end 110.008 73.364924) (width 0.2) (layer "F.Cu") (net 7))
 (segment (start 104.366 68.055256) (end 104.366 75.438) (width 0.2) (layer "F.Cu") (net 5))
 (segment (start 111.158 68.199) (end 110.031 67.072) (width 0.2) (layer "F.Cu") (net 5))
 (segment (start 110.031 67.072) (end 105.349256 67.072) (width 0.2) (layer "F.Cu") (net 5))
 (segment (start 105.349256 67.072) (end 104.366 68.055256) (width 0.2) (layer "F.Cu") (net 5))
 (segment (start 108.966 75.438) (end 107.651256 75.438) (width 0.2) (layer "F.Cu") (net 6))
 (segment (start 107.746256 69.469) (end 106.349256 68.072) (width 0.2) (layer "F.Cu") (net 6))
 (segment (start 104.766 69.24) (end 105.934 68.072) (width 0.2) (layer "F.Cu") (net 6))
 (segment (start 104.766 72.552744) (end 104.766 69.24) (width 0.2) (layer "F.Cu") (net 6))
 (segment (start 111.158 69.469) (end 107.746256 69.469) (width 0.2) (layer "F.Cu") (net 6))
 (segment (start 106.349256 68.072) (end 105.934 68.072) (width 0.2) (layer "F.Cu") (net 6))
 (segment (start 107.651256 75.438) (end 104.766 72.552744) (width 0.2) (layer "F.Cu") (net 6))
 (segment (start 117.308 68.844) (end 119.608 68.844) (width 0.2) (layer "F.Cu") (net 10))
 (segment (start 119.608 70.094) (end 118.963 70.739) (width 0.2) (layer "F.Cu") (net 10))
 (segment (start 113.594 65.13) (end 117.308 68.844) (width 0.2) (layer "F.Cu") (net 10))
 (segment (start 121.682 68.02) (end 118.963 70.739) (width 0.2) (layer "F.Cu") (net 10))
 (segment (start 119.608 68.844) (end 119.608 70.094) (width 0.2) (layer "F.Cu") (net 10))
 (segment (start 113.594 64.77) (end 113.594 65.13) (width 0.2) (layer "F.Cu") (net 10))
 (segment (start 118.963 70.739) (end 118.458 70.739) (width 0.2) (layer "F.Cu") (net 10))
 (segment (start 121.682 67.31) (end 121.682 68.02) (width 0.2) (layer "F.Cu") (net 10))
 (segment (start 118.458 69.469) (end 116.383811 69.469) (width 0.2) (layer "F.Cu") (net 11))
 (segment (start 116.383811 69.469) (end 111.684811 64.77) (width 0.2) (layer "F.Cu") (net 11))
 (segment (start 111.684811 64.77) (end 108.994 64.77) (width 0.2) (layer "F.Cu") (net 11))
 (segment (start 122.682 67.894744) (end 122.682 64.77) (width 0.2) (layer "F.Cu") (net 9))
 (segment (start 122.682 64.77) (end 122.936 64.516) (width 0.2) (layer "F.Cu") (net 9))
 (segment (start 119.825057 72.009) (end 119.825057 70.751687) (width 0.2) (layer "F.Cu") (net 9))
 (segment (start 118.458 72.009) (end 119.825057 72.009) (width 0.2) (layer "F.Cu") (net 9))
 (segment (start 119.825057 70.751687) (end 122.682 67.894744) (width 0.2) (layer "F.Cu") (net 9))
 (via (at 122.936 64.516) (size 0.6) (drill 0.3) (layers "F.Cu" "B.Cu") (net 9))
 (segment (start 122.682 64.77) (end 118.194 64.77) (width 0.2) (layer "B.Cu") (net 9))
 (segment (start 122.936 64.516) (end 122.682 64.77) (width 0.2) (layer "B.Cu") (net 9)))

